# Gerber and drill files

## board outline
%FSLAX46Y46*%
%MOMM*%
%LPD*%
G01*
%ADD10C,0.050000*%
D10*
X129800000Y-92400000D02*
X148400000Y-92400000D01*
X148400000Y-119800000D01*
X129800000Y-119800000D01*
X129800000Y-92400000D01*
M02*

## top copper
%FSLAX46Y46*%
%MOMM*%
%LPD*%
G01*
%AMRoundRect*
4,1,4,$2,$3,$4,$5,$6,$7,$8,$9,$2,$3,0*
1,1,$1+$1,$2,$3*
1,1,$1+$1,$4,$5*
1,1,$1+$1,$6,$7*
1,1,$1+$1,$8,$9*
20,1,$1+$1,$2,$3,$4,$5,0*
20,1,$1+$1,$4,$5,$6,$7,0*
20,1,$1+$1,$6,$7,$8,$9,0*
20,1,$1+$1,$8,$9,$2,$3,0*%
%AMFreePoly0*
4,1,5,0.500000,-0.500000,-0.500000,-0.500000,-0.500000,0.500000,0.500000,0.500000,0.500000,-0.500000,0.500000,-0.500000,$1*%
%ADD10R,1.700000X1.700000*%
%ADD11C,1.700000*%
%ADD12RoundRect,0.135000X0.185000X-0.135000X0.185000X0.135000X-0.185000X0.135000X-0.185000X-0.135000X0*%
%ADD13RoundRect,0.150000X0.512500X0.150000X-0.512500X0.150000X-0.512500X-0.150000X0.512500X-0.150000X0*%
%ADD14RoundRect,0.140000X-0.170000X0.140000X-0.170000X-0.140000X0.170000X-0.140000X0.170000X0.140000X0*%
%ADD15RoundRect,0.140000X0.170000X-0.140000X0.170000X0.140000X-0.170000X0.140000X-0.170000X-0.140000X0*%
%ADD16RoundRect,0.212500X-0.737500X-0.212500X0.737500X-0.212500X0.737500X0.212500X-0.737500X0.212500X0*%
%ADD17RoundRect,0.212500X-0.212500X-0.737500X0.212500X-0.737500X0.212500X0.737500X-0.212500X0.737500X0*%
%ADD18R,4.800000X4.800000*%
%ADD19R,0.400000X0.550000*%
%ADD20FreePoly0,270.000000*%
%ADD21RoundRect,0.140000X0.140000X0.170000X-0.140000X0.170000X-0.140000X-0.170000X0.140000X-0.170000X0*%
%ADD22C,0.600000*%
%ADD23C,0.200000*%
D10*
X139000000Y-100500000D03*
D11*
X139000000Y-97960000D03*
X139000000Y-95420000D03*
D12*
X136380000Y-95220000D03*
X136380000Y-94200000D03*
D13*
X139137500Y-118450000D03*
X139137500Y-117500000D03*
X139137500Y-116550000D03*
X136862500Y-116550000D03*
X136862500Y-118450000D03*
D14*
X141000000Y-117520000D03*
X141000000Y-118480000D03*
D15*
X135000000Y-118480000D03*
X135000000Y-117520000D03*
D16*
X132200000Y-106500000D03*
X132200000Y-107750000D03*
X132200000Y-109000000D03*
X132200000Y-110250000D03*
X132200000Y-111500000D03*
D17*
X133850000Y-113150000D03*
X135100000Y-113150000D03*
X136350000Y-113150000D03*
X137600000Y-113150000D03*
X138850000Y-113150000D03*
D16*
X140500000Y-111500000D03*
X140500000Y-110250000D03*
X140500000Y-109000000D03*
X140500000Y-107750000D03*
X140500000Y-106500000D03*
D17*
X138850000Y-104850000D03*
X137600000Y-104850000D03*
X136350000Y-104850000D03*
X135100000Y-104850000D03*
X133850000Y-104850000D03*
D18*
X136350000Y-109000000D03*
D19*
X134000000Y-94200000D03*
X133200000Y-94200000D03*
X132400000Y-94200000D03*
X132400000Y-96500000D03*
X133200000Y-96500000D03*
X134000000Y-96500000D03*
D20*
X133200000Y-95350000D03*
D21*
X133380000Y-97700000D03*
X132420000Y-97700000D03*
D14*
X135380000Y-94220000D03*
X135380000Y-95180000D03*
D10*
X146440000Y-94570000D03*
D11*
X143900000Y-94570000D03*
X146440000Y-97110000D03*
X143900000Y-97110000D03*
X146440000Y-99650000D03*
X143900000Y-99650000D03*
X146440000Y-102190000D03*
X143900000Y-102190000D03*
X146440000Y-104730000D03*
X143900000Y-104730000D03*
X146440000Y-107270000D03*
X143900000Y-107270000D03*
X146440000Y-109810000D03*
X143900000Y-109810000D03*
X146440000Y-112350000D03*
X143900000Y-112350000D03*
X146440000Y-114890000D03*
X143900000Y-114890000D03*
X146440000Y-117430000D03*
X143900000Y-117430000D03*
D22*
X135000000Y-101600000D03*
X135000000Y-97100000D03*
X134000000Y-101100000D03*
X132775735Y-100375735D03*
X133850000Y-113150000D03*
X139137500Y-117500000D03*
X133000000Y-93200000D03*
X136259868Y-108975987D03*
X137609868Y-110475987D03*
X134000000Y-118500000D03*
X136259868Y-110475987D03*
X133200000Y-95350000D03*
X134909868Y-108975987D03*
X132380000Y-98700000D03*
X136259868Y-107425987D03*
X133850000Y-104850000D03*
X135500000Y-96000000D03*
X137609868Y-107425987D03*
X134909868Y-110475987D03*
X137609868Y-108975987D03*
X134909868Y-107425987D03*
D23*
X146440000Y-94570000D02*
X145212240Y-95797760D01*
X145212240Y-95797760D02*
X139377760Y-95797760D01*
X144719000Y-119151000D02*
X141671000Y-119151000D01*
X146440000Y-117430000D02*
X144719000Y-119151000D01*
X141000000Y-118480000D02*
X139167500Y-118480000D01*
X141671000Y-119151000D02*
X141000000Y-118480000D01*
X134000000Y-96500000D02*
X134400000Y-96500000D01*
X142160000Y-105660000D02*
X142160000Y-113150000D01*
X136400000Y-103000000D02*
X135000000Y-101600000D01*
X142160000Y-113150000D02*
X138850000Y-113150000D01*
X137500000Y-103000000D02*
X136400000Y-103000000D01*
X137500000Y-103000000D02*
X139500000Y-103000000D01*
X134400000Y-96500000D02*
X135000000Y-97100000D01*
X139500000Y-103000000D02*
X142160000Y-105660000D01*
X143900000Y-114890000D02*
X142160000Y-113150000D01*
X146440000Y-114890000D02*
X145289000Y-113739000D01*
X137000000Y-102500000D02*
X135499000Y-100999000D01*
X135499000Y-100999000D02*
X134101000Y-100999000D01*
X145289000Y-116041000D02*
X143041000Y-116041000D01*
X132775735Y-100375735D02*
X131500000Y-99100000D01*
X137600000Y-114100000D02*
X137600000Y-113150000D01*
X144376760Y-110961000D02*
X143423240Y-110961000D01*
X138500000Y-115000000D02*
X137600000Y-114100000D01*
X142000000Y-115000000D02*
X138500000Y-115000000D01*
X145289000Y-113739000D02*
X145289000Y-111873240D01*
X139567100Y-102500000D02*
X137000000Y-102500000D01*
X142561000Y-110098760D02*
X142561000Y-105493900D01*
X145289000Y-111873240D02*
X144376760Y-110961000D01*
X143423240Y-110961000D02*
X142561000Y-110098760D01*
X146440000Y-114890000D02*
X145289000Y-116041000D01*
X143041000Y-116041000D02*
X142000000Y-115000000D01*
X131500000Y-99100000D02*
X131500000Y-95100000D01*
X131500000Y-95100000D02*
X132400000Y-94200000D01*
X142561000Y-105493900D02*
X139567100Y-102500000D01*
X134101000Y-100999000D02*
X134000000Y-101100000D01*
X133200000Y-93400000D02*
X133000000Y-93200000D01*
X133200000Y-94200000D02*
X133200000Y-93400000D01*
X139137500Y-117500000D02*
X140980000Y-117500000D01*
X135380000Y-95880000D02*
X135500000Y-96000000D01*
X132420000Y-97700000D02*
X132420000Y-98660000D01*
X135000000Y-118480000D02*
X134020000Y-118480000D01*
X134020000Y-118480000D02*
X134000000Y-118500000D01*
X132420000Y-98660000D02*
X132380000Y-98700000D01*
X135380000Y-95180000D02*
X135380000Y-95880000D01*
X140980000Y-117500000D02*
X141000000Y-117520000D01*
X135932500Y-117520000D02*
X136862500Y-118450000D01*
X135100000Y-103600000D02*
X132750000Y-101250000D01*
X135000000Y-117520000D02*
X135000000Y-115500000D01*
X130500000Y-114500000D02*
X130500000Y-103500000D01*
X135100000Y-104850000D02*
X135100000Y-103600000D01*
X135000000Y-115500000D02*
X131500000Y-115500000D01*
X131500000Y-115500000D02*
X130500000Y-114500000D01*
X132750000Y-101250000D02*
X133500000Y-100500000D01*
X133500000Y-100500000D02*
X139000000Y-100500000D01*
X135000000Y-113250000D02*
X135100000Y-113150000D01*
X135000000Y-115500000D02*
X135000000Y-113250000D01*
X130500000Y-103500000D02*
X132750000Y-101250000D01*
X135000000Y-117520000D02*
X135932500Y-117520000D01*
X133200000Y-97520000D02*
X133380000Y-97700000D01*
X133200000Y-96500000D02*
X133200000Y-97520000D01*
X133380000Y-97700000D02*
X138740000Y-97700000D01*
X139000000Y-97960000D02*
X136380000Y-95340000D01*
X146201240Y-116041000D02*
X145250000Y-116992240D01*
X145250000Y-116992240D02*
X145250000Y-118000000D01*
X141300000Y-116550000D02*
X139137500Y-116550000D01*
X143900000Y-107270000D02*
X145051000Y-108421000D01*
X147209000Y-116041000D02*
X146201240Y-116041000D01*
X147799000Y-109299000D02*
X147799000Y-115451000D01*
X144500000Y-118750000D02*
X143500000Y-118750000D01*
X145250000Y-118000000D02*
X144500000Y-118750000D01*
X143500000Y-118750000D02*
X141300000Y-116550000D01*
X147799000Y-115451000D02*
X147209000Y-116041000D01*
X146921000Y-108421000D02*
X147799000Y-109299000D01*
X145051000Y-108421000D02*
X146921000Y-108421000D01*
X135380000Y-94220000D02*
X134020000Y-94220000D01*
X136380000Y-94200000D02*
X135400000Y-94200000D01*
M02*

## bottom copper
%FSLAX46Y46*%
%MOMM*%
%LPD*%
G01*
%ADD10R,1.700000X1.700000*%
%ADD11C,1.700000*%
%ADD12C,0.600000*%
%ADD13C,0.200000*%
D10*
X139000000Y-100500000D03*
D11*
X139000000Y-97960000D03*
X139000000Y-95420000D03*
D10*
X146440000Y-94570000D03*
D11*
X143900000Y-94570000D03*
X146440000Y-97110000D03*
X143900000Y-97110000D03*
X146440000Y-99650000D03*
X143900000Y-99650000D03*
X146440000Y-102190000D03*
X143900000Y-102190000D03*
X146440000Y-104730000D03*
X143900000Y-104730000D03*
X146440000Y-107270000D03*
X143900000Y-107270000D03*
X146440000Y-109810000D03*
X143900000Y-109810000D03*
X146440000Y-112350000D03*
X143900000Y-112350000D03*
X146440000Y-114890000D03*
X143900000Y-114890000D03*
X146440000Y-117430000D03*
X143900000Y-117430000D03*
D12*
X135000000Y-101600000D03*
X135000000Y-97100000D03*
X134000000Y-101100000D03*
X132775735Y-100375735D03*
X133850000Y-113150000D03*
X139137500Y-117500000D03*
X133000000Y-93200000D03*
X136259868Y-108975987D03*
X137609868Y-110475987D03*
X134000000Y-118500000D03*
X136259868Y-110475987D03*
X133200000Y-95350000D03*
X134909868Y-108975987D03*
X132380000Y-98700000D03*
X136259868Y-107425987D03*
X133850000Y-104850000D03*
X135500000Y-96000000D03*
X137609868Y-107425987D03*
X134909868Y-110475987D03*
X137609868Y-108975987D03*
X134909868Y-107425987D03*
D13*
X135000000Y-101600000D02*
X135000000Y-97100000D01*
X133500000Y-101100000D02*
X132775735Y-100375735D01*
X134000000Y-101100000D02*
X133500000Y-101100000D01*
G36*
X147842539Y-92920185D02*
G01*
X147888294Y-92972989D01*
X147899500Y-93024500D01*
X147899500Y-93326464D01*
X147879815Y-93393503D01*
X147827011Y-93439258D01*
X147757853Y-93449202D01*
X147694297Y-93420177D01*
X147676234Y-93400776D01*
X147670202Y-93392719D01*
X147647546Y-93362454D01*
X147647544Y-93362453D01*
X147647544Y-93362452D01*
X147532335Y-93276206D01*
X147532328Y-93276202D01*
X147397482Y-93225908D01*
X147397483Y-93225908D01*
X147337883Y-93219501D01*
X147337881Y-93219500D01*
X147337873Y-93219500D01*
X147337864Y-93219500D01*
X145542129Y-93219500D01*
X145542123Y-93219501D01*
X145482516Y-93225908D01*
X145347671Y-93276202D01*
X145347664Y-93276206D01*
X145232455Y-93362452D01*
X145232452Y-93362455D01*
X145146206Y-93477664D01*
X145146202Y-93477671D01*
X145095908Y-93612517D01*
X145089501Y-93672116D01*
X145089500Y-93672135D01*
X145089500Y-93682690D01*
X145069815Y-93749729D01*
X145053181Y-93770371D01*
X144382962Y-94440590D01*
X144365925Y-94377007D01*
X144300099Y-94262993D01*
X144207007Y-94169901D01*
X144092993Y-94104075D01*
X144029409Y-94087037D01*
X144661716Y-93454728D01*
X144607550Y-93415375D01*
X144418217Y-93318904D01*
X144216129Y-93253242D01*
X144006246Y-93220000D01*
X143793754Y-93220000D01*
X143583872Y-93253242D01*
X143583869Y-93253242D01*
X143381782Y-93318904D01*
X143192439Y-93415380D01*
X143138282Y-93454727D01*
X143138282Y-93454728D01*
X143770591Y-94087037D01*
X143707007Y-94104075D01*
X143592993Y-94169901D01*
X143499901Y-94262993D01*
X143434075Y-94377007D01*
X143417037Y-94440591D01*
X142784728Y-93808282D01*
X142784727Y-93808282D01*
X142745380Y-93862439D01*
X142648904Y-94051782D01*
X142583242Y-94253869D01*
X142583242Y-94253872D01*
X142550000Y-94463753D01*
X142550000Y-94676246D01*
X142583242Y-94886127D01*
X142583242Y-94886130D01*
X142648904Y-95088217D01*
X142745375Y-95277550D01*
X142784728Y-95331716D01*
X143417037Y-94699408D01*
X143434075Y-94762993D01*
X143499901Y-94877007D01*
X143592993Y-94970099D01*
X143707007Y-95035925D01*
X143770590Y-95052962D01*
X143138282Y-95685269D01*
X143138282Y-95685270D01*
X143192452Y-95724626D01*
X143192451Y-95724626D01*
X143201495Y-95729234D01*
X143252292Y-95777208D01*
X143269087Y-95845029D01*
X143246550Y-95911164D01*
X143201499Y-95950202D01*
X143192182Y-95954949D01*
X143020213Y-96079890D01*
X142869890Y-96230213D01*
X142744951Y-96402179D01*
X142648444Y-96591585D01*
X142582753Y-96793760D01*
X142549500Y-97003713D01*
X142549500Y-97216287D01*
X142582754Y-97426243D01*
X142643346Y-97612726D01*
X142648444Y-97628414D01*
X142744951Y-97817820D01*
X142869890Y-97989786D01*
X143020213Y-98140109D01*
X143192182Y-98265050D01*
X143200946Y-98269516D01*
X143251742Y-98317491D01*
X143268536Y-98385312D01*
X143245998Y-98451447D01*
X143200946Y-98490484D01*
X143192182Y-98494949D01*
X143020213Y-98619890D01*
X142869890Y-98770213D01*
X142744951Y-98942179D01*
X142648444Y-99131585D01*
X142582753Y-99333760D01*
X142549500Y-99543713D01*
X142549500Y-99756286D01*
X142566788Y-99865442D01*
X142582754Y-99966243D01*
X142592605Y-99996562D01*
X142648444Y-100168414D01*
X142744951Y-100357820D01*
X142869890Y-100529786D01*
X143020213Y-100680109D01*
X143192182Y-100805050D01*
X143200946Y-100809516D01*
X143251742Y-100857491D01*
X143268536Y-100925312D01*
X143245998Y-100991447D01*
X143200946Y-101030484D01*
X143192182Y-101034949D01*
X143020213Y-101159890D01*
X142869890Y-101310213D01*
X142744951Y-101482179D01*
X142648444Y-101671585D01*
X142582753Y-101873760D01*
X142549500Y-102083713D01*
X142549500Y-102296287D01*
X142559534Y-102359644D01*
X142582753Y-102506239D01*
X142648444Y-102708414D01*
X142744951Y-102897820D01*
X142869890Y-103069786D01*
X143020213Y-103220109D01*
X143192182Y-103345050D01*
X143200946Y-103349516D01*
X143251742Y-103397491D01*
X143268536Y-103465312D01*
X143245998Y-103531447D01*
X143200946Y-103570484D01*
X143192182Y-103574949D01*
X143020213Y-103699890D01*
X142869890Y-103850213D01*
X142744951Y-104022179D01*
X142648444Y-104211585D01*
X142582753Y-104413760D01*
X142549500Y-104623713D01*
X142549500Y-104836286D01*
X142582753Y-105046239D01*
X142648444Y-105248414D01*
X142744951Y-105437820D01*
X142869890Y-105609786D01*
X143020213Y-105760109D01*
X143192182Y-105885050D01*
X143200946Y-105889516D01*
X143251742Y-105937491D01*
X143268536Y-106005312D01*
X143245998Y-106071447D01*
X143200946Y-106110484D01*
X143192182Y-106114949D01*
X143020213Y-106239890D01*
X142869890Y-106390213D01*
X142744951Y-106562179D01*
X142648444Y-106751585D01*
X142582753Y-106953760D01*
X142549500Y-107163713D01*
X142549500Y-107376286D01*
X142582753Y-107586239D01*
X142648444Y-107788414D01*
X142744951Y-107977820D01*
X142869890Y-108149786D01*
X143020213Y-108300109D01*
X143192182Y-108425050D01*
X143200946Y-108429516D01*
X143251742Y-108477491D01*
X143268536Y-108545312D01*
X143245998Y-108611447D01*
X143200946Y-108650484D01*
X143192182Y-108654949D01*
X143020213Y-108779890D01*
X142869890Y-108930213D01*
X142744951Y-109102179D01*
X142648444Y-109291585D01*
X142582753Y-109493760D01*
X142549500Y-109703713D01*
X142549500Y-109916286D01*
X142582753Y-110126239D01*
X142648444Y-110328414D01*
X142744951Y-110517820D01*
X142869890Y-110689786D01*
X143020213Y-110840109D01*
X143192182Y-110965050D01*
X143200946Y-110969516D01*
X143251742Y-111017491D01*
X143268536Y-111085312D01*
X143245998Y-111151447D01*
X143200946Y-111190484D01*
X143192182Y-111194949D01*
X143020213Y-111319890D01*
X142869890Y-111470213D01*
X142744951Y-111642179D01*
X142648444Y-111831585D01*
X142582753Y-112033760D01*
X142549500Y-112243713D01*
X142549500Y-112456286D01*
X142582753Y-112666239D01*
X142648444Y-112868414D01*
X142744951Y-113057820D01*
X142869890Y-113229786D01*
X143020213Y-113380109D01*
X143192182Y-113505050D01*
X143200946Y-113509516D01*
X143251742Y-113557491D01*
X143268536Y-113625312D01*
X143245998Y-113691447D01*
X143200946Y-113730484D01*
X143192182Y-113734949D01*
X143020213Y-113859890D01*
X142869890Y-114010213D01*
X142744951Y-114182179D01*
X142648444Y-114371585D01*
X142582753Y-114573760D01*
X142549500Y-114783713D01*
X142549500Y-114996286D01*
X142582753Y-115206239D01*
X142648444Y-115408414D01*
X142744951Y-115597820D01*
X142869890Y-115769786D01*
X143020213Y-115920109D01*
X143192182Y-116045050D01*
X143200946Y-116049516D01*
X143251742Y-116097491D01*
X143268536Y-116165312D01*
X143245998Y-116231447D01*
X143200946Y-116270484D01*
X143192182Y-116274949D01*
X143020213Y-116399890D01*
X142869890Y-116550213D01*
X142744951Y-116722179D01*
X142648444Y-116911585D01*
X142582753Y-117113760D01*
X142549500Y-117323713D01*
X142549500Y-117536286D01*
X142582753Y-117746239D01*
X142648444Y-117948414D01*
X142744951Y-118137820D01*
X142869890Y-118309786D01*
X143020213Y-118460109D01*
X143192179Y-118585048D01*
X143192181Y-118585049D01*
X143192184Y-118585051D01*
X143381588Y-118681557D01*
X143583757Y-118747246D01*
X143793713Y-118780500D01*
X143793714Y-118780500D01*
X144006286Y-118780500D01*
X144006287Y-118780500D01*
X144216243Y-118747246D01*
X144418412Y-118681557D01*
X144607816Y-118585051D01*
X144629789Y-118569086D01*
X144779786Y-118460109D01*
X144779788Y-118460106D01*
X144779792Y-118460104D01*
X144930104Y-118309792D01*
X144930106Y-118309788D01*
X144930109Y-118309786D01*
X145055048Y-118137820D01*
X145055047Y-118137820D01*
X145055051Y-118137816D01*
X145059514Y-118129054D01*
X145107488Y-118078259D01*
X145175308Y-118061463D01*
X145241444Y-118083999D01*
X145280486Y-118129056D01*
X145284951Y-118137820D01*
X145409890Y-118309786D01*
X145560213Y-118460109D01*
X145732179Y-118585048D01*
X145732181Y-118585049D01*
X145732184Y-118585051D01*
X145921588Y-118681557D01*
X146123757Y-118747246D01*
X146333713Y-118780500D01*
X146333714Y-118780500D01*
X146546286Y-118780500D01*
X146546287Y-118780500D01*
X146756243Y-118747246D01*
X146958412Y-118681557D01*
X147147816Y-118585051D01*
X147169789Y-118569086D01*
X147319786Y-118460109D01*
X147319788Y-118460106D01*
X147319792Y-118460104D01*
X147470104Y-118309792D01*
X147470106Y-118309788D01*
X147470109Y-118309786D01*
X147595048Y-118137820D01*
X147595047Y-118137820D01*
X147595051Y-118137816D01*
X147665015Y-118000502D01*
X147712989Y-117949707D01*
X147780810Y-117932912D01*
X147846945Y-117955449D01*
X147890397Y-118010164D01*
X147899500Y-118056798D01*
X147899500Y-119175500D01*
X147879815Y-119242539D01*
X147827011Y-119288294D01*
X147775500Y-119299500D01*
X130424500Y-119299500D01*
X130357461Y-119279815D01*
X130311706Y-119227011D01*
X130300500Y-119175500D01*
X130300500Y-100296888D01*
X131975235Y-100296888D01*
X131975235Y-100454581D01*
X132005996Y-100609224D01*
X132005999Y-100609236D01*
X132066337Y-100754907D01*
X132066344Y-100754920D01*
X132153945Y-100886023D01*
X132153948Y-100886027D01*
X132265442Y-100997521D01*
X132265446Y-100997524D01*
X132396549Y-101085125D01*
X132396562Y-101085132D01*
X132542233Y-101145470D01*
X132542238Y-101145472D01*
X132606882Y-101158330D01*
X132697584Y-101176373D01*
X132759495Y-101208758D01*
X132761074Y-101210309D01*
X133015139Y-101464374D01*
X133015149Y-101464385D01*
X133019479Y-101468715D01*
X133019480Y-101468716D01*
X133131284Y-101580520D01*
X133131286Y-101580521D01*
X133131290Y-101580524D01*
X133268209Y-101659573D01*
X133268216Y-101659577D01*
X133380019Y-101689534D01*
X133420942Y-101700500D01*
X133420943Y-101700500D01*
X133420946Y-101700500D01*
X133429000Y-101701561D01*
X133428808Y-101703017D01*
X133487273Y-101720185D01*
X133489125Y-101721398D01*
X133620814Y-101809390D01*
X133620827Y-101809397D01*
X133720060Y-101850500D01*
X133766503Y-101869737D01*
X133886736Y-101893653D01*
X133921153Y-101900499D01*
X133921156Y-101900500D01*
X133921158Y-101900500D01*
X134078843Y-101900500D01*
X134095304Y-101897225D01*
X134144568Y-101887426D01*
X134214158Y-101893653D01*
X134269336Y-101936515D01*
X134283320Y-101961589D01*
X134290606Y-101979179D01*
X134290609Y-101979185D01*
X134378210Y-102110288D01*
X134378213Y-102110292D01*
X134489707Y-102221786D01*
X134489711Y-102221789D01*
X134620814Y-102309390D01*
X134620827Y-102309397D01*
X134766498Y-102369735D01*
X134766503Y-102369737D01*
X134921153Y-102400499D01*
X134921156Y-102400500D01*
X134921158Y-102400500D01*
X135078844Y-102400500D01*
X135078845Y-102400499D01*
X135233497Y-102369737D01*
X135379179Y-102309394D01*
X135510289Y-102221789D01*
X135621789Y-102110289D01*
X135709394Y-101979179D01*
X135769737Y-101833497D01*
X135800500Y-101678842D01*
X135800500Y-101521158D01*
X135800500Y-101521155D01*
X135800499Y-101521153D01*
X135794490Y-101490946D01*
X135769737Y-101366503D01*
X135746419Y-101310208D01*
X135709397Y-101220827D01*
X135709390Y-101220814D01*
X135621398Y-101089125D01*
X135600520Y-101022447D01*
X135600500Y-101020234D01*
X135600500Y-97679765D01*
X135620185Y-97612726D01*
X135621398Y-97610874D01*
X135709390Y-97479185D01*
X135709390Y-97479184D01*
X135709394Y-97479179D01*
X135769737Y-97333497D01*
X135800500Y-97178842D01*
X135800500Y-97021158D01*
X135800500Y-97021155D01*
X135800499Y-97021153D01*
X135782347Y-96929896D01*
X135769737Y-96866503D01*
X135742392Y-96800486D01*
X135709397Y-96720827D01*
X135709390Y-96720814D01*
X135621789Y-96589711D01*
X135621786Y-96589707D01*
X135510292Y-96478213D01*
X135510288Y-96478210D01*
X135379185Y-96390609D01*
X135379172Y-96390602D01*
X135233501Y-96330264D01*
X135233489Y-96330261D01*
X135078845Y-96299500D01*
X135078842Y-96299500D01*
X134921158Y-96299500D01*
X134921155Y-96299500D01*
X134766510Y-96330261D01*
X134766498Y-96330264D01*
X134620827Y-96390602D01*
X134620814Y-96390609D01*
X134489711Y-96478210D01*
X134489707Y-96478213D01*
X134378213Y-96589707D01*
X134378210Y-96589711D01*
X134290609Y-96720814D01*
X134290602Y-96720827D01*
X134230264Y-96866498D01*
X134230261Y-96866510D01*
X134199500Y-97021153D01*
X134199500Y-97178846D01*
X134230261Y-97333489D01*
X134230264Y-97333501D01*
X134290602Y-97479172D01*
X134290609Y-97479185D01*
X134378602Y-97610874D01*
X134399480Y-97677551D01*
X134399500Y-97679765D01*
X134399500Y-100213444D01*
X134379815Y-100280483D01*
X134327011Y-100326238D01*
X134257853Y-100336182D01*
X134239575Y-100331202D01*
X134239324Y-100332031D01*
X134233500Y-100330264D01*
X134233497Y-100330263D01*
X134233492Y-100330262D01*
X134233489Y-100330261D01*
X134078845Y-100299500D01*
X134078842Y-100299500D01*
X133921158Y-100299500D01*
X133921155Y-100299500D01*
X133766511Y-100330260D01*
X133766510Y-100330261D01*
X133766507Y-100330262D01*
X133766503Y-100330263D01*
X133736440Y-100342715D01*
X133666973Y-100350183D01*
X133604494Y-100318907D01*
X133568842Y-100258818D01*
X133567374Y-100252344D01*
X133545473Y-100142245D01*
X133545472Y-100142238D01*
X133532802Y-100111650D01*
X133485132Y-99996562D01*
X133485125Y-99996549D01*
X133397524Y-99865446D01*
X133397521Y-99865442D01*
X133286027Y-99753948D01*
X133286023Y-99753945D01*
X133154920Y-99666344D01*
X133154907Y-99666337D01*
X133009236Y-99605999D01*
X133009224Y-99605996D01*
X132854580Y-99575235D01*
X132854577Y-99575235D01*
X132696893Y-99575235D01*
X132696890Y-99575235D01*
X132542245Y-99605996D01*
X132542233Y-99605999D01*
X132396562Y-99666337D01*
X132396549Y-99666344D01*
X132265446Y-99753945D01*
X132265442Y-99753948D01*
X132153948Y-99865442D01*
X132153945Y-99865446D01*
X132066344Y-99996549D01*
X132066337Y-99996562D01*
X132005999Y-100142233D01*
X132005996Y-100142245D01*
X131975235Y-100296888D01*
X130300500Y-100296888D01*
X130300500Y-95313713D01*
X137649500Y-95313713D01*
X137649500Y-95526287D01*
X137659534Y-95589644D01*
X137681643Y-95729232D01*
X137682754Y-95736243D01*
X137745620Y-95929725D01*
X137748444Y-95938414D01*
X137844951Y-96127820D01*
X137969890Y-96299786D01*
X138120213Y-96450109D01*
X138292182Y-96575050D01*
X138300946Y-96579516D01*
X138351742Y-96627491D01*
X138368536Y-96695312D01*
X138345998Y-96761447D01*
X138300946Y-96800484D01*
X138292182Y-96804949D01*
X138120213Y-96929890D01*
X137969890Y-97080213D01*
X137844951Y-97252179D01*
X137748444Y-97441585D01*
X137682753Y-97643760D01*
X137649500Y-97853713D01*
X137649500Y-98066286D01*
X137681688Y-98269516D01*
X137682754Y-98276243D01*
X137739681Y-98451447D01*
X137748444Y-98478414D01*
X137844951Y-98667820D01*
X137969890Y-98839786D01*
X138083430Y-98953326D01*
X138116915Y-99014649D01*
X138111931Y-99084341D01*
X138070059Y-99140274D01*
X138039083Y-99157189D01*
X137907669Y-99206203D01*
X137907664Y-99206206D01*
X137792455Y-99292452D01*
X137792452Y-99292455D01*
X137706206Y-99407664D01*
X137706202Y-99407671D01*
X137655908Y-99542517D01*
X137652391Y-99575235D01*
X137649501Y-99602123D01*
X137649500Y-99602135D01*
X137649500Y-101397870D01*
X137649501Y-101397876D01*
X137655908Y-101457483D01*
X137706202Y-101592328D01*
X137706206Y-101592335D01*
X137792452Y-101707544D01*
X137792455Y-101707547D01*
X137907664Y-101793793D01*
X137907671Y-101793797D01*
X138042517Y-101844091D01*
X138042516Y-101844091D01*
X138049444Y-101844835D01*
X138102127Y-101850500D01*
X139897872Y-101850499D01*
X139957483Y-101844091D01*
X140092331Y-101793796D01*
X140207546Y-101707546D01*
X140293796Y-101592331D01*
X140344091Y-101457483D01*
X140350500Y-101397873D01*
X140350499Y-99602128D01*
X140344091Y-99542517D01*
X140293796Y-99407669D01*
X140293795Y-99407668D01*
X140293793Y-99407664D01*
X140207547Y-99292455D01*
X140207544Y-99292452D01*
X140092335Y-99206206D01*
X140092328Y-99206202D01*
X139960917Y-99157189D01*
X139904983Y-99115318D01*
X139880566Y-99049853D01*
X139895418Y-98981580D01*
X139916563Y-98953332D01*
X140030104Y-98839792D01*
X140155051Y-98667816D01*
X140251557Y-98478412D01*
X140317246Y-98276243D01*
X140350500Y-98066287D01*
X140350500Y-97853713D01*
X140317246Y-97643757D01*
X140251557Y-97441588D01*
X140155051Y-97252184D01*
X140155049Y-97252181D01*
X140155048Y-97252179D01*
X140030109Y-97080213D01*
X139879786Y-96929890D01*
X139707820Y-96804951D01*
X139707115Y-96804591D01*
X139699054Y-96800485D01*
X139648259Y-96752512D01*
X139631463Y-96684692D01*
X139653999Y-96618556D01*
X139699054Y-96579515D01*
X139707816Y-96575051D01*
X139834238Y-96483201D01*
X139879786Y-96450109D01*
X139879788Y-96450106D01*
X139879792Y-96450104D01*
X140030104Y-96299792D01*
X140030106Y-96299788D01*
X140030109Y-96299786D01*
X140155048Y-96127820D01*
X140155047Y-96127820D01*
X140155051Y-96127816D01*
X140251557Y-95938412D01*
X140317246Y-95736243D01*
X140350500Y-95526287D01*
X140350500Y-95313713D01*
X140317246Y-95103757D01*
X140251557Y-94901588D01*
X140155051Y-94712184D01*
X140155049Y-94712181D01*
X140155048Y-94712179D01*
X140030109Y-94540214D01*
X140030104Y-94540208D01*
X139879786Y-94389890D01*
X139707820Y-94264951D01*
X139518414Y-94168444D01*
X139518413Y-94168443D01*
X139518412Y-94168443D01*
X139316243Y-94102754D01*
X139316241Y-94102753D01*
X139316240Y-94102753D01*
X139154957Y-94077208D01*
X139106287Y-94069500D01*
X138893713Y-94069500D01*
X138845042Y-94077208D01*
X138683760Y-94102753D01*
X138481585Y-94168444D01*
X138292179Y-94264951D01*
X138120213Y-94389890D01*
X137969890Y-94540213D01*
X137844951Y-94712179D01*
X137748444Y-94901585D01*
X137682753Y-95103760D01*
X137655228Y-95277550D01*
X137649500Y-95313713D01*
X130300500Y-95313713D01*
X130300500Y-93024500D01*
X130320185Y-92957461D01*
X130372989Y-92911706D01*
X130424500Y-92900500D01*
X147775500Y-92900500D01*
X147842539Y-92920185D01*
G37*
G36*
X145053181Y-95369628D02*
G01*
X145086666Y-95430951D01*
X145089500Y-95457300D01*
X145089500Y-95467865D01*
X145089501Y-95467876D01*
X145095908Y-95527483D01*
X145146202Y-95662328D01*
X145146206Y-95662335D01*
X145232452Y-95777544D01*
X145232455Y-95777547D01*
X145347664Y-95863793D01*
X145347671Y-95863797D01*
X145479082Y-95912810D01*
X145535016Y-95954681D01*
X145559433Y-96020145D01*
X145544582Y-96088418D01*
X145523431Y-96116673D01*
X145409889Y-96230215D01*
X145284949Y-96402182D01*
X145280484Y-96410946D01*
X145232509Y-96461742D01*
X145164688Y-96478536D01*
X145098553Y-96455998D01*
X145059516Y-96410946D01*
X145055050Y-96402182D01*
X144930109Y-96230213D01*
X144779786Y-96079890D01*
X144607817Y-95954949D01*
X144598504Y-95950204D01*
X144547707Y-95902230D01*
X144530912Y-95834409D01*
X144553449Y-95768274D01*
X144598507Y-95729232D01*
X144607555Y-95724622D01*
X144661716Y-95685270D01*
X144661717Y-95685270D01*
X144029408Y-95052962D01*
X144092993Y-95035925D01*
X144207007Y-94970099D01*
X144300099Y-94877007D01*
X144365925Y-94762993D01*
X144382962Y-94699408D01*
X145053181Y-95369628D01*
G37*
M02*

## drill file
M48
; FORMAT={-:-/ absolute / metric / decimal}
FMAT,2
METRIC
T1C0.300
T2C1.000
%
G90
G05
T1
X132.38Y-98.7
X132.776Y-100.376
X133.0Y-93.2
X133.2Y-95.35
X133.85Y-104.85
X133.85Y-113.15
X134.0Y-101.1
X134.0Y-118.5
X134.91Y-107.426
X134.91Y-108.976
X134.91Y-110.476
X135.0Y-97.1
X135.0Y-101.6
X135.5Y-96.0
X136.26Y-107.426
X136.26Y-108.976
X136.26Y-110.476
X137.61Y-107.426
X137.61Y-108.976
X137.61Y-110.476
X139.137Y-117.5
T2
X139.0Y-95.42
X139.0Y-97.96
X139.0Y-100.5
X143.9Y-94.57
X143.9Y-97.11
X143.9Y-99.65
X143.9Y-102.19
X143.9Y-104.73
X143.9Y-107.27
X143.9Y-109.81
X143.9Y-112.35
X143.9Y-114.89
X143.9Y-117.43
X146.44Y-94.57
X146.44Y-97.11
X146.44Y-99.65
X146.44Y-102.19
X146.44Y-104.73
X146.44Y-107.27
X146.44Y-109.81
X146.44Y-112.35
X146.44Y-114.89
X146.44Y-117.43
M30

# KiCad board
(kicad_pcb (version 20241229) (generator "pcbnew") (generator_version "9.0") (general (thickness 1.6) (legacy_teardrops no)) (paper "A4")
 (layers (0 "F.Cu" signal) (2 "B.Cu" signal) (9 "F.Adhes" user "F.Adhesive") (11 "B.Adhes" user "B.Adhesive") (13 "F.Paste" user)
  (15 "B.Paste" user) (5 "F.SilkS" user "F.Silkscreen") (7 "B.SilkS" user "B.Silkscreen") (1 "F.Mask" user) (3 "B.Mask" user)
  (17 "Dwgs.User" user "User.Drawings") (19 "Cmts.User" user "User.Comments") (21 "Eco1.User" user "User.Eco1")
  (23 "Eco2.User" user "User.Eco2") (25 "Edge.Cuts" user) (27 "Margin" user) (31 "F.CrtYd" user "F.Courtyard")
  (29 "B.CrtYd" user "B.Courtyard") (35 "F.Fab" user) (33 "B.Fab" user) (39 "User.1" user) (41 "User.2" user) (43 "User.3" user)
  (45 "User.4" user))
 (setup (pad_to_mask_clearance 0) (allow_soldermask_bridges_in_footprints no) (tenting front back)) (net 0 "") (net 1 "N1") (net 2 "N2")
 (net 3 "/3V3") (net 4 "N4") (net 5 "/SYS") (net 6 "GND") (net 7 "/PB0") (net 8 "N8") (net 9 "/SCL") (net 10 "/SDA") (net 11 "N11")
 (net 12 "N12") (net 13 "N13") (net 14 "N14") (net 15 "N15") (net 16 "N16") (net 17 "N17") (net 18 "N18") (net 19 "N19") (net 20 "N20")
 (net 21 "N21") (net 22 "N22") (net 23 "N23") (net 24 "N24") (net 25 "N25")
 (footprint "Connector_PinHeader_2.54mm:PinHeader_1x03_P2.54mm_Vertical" (layer "F.Cu") (at 139 100.5 180)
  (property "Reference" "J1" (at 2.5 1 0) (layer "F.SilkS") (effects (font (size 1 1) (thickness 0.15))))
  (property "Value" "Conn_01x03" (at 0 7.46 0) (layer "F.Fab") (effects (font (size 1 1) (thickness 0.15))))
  (pad "1" thru_hole rect (at 0 0 180) (size 1.7 1.7) (drill 1) (layers "*.Cu" "*.Mask") (remove_unused_layers no) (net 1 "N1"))
  (pad "2" thru_hole circle (at 0 2.54 180) (size 1.7 1.7) (drill 1) (layers "*.Cu" "*.Mask") (remove_unused_layers no) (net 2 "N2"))
  (pad "3" thru_hole circle (at 0 5.08 180) (size 1.7 1.7) (drill 1) (layers "*.Cu" "*.Mask") (remove_unused_layers no) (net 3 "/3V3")))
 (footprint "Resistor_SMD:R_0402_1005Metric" (layer "F.Cu") (at 136.38 94.71 90)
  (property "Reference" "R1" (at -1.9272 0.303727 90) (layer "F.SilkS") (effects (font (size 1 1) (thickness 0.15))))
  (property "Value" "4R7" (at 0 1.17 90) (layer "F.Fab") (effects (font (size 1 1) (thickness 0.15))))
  (pad "1" smd roundrect (at -0.51 0 90) (size 0.54 0.64) (layers "F.Cu" "F.Mask" "F.Paste") (roundrect_rratio 0.25) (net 2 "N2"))
  (pad "2" smd roundrect (at 0.51 0 90) (size 0.54 0.64) (layers "F.Cu" "F.Mask" "F.Paste") (roundrect_rratio 0.25) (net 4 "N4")))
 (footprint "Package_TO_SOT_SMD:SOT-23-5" (layer "F.Cu") (at 138 117.5 180)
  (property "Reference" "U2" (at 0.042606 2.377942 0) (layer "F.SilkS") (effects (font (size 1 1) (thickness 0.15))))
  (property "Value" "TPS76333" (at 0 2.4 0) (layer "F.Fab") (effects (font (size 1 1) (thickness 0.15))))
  (pad "1" smd roundrect (at -1.1375 -0.95 180) (size 1.325 0.6) (layers "F.Cu" "F.Mask" "F.Paste") (roundrect_rratio 0.25) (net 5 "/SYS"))
  (pad "2" smd roundrect (at -1.1375 0 180) (size 1.325 0.6) (layers "F.Cu" "F.Mask" "F.Paste") (roundrect_rratio 0.25) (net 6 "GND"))
  (pad "3" smd roundrect (at -1.1375 0.95 180) (size 1.325 0.6) (layers "F.Cu" "F.Mask" "F.Paste") (roundrect_rratio 0.25) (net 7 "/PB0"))
  (pad "4" smd roundrect (at 1.1375 0.95 180) (size 1.325 0.6) (layers "F.Cu" "F.Mask" "F.Paste") (roundrect_rratio 0.25) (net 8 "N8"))
  (pad "5" smd roundrect (at 1.1375 -0.95 180) (size 1.325 0.6) (layers "F.Cu" "F.Mask" "F.Paste") (roundrect_rratio 0.25) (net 1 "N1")))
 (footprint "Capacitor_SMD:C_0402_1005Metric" (layer "F.Cu") (at 141 118 -90)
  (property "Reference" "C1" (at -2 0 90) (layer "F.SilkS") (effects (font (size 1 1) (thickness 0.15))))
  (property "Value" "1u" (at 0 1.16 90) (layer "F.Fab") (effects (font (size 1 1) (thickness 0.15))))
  (pad "1" smd roundrect (at -0.48 0 270) (size 0.56 0.62) (layers "F.Cu" "F.Mask" "F.Paste") (roundrect_rratio 0.25) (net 6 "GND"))
  (pad "2" smd roundrect (at 0.48 0 270) (size 0.56 0.62) (layers "F.Cu" "F.Mask" "F.Paste") (roundrect_rratio 0.25) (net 5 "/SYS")))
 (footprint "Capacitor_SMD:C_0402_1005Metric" (layer "F.Cu") (at 135 118 90)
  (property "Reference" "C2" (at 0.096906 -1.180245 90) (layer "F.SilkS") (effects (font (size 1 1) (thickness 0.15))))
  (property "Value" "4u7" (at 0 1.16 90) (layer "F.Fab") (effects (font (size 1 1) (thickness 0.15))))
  (pad "1" smd roundrect (at -0.48 0 90) (size 0.56 0.62) (layers "F.Cu" "F.Mask" "F.Paste") (roundrect_rratio 0.25) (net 6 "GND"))
  (pad "2" smd roundrect (at 0.48 0 90) (size 0.56 0.62) (layers "F.Cu" "F.Mask" "F.Paste") (roundrect_rratio 0.25) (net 1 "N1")))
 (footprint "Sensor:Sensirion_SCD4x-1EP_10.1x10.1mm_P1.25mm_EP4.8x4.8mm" (layer "F.Cu") (at 136.35 109)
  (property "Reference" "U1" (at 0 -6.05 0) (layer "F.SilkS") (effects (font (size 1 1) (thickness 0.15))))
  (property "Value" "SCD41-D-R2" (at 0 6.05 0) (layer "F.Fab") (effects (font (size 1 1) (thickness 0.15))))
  (pad "" smd roundrect (at -1.2 -1.2) (size 1.93 1.93) (layers "F.Paste") (roundrect_rratio 0.129534))
  (pad "" smd roundrect (at -1.2 1.2) (size 1.93 1.93) (layers "F.Paste") (roundrect_rratio 0.129534))
  (pad "" smd roundrect (at 1.2 -1.2) (size 1.93 1.93) (layers "F.Paste") (roundrect_rratio 0.129534))
  (pad "" smd roundrect (at 1.2 1.2) (size 1.93 1.93) (layers "F.Paste") (roundrect_rratio 0.129534))
  (pad "1" smd roundrect (at -4.15 -2.5) (size 1.9 0.85) (layers "F.Cu" "F.Mask" "F.Paste") (roundrect_rratio 0.25))
  (pad "2" smd roundrect (at -4.15 -1.25) (size 1.9 0.85) (layers "F.Cu" "F.Mask" "F.Paste") (roundrect_rratio 0.25))
  (pad "3" smd roundrect (at -4.15 0) (size 1.9 0.85) (layers "F.Cu" "F.Mask" "F.Paste") (roundrect_rratio 0.25))
  (pad "4" smd roundrect (at -4.15 1.25) (size 1.9 0.85) (layers "F.Cu" "F.Mask" "F.Paste") (roundrect_rratio 0.25))
  (pad "5" smd roundrect (at -4.15 2.5) (size 1.9 0.85) (layers "F.Cu" "F.Mask" "F.Paste") (roundrect_rratio 0.25))
  (pad "6" smd roundrect (at -2.5 4.15) (size 0.85 1.9) (layers "F.Cu" "F.Mask" "F.Paste") (roundrect_rratio 0.25) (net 6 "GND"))
  (pad "7" smd roundrect (at -1.25 4.15) (size 0.85 1.9) (layers "F.Cu" "F.Mask" "F.Paste") (roundrect_rratio 0.25) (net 1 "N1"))
  (pad "8" smd roundrect (at 0 4.15) (size 0.85 1.9) (layers "F.Cu" "F.Mask" "F.Paste") (roundrect_rratio 0.25))
  (pad "9" smd roundrect (at 1.25 4.15) (size 0.85 1.9) (layers "F.Cu" "F.Mask" "F.Paste") (roundrect_rratio 0.25) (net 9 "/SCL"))
  (pad "10" smd roundrect (at 2.5 4.15) (size 0.85 1.9) (layers "F.Cu" "F.Mask" "F.Paste") (roundrect_rratio 0.25) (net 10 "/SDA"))
  (pad "11" smd roundrect (at 4.15 2.5) (size 1.9 0.85) (layers "F.Cu" "F.Mask" "F.Paste") (roundrect_rratio 0.25))
  (pad "12" smd roundrect (at 4.15 1.25) (size 1.9 0.85) (layers "F.Cu" "F.Mask" "F.Paste") (roundrect_rratio 0.25))
  (pad "13" smd roundrect (at 4.15 0) (size 1.9 0.85) (layers "F.Cu" "F.Mask" "F.Paste") (roundrect_rratio 0.25))
  (pad "14" smd roundrect (at 4.15 -1.25) (size 1.9 0.85) (layers "F.Cu" "F.Mask" "F.Paste") (roundrect_rratio 0.25))
  (pad "15" smd roundrect (at 4.15 -2.5) (size 1.9 0.85) (layers "F.Cu" "F.Mask" "F.Paste") (roundrect_rratio 0.25))
  (pad "16" smd roundrect (at 2.5 -4.15) (size 0.85 1.9) (layers "F.Cu" "F.Mask" "F.Paste") (roundrect_rratio 0.25))
  (pad "17" smd roundrect (at 1.25 -4.15) (size 0.85 1.9) (layers "F.Cu" "F.Mask" "F.Paste") (roundrect_rratio 0.25))
  (pad "18" smd roundrect (at 0 -4.15) (size 0.85 1.9) (layers "F.Cu" "F.Mask" "F.Paste") (roundrect_rratio 0.25))
  (pad "19" smd roundrect (at -1.25 -4.15) (size 0.85 1.9) (layers "F.Cu" "F.Mask" "F.Paste") (roundrect_rratio 0.25) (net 1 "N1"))
  (pad "20" smd roundrect (at -2.5 -4.15) (size 0.85 1.9) (layers "F.Cu" "F.Mask" "F.Paste") (roundrect_rratio 0.25) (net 6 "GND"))
  (pad "21" smd rect (at 0 0) (size 4.8 4.8) (layers "F.Cu" "F.Mask") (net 6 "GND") (zone_connect 2)))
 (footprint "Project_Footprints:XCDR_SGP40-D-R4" (layer "F.Cu") (at 133.2 95.35 -90)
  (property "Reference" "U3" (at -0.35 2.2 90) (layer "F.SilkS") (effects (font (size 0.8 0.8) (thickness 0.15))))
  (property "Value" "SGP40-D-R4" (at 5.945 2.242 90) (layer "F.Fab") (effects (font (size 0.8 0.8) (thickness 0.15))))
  (pad "1" smd rect (at -1.15 -0.8 270) (size 0.55 0.4) (layers "F.Cu" "F.Mask" "F.Paste") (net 4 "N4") (solder_mask_margin 0.102))
  (pad "2" smd rect (at -1.15 0 270) (size 0.55 0.4) (layers "F.Cu" "F.Mask" "F.Paste") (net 6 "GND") (solder_mask_margin 0.102))
  (pad "3" smd rect (at -1.15 0.8 270) (size 0.55 0.4) (layers "F.Cu" "F.Mask" "F.Paste") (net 9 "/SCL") (solder_mask_margin 0.102))
  (pad "4" smd rect (at 1.15 0.8 270) (size 0.55 0.4) (layers "F.Cu" "F.Mask" "F.Paste") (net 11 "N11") (solder_mask_margin 0.102))
  (pad "5" smd rect (at 1.15 0 270) (size 0.55 0.4) (layers "F.Cu" "F.Mask" "F.Paste") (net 2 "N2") (solder_mask_margin 0.102))
  (pad "6" smd rect (at 1.15 -0.8 270) (size 0.55 0.4) (layers "F.Cu" "F.Mask" "F.Paste") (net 10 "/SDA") (solder_mask_margin 0.102))
  (pad "7" smd custom (at 0 0 270) (size 1 1) (layers "F.Cu") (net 6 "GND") (options (clearance outline) (anchor rect)) (primitives)))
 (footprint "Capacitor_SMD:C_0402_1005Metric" (layer "F.Cu") (at 132.9 97.7 180)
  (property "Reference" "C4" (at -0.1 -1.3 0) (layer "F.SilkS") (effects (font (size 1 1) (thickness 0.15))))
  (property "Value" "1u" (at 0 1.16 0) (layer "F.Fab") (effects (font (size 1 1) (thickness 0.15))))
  (pad "1" smd roundrect (at -0.48 0 180) (size 0.56 0.62) (layers "F.Cu" "F.Mask" "F.Paste") (roundrect_rratio 0.25) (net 2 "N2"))
  (pad "2" smd roundrect (at 0.48 0 180) (size 0.56 0.62) (layers "F.Cu" "F.Mask" "F.Paste") (roundrect_rratio 0.25) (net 6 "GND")))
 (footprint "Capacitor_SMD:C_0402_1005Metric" (layer "F.Cu") (at 135.38 94.7 -90)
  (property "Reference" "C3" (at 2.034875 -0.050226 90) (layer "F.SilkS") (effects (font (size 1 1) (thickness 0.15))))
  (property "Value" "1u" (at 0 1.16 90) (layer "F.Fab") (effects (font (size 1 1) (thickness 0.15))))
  (pad "1" smd roundrect (at -0.48 0 270) (size 0.56 0.62) (layers "F.Cu" "F.Mask" "F.Paste") (roundrect_rratio 0.25) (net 4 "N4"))
  (pad "2" smd roundrect (at 0.48 0 270) (size 0.56 0.62) (layers "F.Cu" "F.Mask" "F.Paste") (roundrect_rratio 0.25) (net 6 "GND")))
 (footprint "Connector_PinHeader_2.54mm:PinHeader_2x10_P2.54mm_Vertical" (layer "B.Cu") (at 146.44 94.57 180)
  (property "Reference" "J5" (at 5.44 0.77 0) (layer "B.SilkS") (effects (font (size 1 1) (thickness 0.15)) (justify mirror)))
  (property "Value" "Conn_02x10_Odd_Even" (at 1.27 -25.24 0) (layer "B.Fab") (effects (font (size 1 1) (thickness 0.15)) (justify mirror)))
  (pad "1" thru_hole rect (at 0 0 180) (size 1.7 1.7) (drill 1) (layers "*.Cu" "*.Mask") (remove_unused_layers no) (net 3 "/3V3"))
  (pad "2" thru_hole circle (at 2.54 0 180) (size 1.7 1.7) (drill 1) (layers "*.Cu" "*.Mask") (remove_unused_layers no) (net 6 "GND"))
  (pad "3" thru_hole circle (at 0 -2.54 180) (size 1.7 1.7) (drill 1) (layers "*.Cu" "*.Mask") (remove_unused_layers no) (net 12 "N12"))
  (pad "4" thru_hole circle (at 2.54 -2.54 180) (size 1.7 1.7) (drill 1) (layers "*.Cu" "*.Mask") (remove_unused_layers no) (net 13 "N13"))
  (pad "5" thru_hole circle (at 0 -5.08 180) (size 1.7 1.7) (drill 1) (layers "*.Cu" "*.Mask") (remove_unused_layers no) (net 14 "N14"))
  (pad "6" thru_hole circle (at 2.54 -5.08 180) (size 1.7 1.7) (drill 1) (layers "*.Cu" "*.Mask") (remove_unused_layers no) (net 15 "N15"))
  (pad "7" thru_hole circle (at 0 -7.62 180) (size 1.7 1.7) (drill 1) (layers "*.Cu" "*.Mask") (remove_unused_layers no) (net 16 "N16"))
  (pad "8" thru_hole circle (at 2.54 -7.62 180) (size 1.7 1.7) (drill 1) (layers "*.Cu" "*.Mask") (remove_unused_layers no) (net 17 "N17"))
  (pad "9" thru_hole circle (at 0 -10.16 180) (size 1.7 1.7) (drill 1) (layers "*.Cu" "*.Mask") (remove_unused_layers no) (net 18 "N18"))
  (pad "10" thru_hole circle (at 2.54 -10.16 180) (size 1.7 1.7) (drill 1) (layers "*.Cu" "*.Mask") (remove_unused_layers no) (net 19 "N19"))
  (pad "11" thru_hole circle (at 0 -12.7 180) (size 1.7 1.7) (drill 1) (layers "*.Cu" "*.Mask") (remove_unused_layers no) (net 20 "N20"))
  (pad "12" thru_hole circle (at 2.54 -12.7 180) (size 1.7 1.7) (drill 1) (layers "*.Cu" "*.Mask") (remove_unused_layers no) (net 7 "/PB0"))
  (pad "13" thru_hole circle (at 0 -15.24 180) (size 1.7 1.7) (drill 1) (layers "*.Cu" "*.Mask") (remove_unused_layers no) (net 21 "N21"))
  (pad "14" thru_hole circle (at 2.54 -15.24 180) (size 1.7 1.7) (drill 1) (layers "*.Cu" "*.Mask") (remove_unused_layers no) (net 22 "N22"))
  (pad "15" thru_hole circle (at 0 -17.78 180) (size 1.7 1.7) (drill 1) (layers "*.Cu" "*.Mask") (remove_unused_layers no) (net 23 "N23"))
  (pad "16" thru_hole circle (at 2.54 -17.78 180) (size 1.7 1.7) (drill 1) (layers "*.Cu" "*.Mask") (remove_unused_layers no) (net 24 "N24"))
  (pad "17" thru_hole circle (at 0 -20.32 180) (size 1.7 1.7) (drill 1) (layers "*.Cu" "*.Mask") (remove_unused_layers no) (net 9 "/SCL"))
  (pad "18" thru_hole circle (at 2.54 -20.32 180) (size 1.7 1.7) (drill 1) (layers "*.Cu" "*.Mask") (remove_unused_layers no)
   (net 10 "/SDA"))
  (pad "19" thru_hole circle (at 0 -22.86 180) (size 1.7 1.7) (drill 1) (layers "*.Cu" "*.Mask") (remove_unused_layers no) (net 5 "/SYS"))
  (pad "20" thru_hole circle (at 2.54 -22.86 180) (size 1.7 1.7) (drill 1) (layers "*.Cu" "*.Mask") (remove_unused_layers no) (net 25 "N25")))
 (gr_rect (start 129.8 92.4) (end 148.4 119.8) (stroke (width 0.05) (type default)) (fill no) (layer "Edge.Cuts"))
 (segment (start 146.44 94.57) (end 145.21224 95.79776) (width 0.2) (layer "F.Cu") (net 3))
 (segment (start 145.21224 95.79776) (end 139.37776 95.79776) (width 0.2) (layer "F.Cu") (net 3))
 (segment (start 144.719 119.151) (end 141.671 119.151) (width 0.2) (layer "F.Cu") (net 5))
 (segment (start 146.44 117.43) (end 144.719 119.151) (width 0.2) (layer "F.Cu") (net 5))
 (segment (start 141 118.48) (end 139.1675 118.48) (width 0.2) (layer "F.Cu") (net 5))
 (segment (start 141.671 119.151) (end 141 118.48) (width 0.2) (layer "F.Cu") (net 5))
 (segment (start 134 96.5) (end 134.4 96.5) (width 0.2) (layer "F.Cu") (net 10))
 (segment (start 142.16 105.66) (end 142.16 113.15) (width 0.2) (layer "F.Cu") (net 10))
 (segment (start 136.4 103) (end 135 101.6) (width 0.2) (layer "F.Cu") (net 10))
 (segment (start 142.16 113.15) (end 138.85 113.15) (width 0.2) (layer "F.Cu") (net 10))
 (segment (start 137.5 103) (end 136.4 103) (width 0.2) (layer "F.Cu") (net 10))
 (segment (start 137.5 103) (end 139.5 103) (width 0.2) (layer "F.Cu") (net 10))
 (segment (start 134.4 96.5) (end 135 97.1) (width 0.2) (layer "F.Cu") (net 10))
 (segment (start 139.5 103) (end 142.16 105.66) (width 0.2) (layer "F.Cu") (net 10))
 (segment (start 143.9 114.89) (end 142.16 113.15) (width 0.2) (layer "F.Cu") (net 10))
 (via (at 135 101.6) (size 0.6) (drill 0.3) (layers "F.Cu" "B.Cu") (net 10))
 (via (at 135 97.1) (size 0.6) (drill 0.3) (layers "F.Cu" "B.Cu") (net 10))
 (segment (start 135 101.6) (end 135 97.1) (width 0.2) (layer "B.Cu") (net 10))
 (segment (start 146.44 114.89) (end 145.289 113.739) (width 0.2) (layer "F.Cu") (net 9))
 (segment (start 137 102.5) (end 135.499 100.999) (width 0.2) (layer "F.Cu") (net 9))
 (segment (start 135.499 100.999) (end 134.101 100.999) (width 0.2) (layer "F.Cu") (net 9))
 (segment (start 145.289 116.041) (end 143.041 116.041) (width 0.2) (layer "F.Cu") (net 9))
 (segment (start 132.775735 100.375735) (end 131.5 99.1) (width 0.2) (layer "F.Cu") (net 9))
 (segment (start 137.6 114.1) (end 137.6 113.15) (width 0.2) (layer "F.Cu") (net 9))
 (segment (start 144.37676 110.961) (end 143.42324 110.961) (width 0.2) (layer "F.Cu") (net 9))
 (segment (start 138.5 115) (end 137.6 114.1) (width 0.2) (layer "F.Cu") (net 9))
 (segment (start 142 115) (end 138.5 115) (width 0.2) (layer "F.Cu") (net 9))
 (segment (start 145.289 113.739) (end 145.289 111.87324) (width 0.2) (layer "F.Cu") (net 9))
 (segment (start 139.5671 102.5) (end 137 102.5) (width 0.2) (layer "F.Cu") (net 9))
 (segment (start 142.561 110.09876) (end 142.561 105.4939) (width 0.2) (layer "F.Cu") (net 9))
 (segment (start 145.289 111.87324) (end 144.37676 110.961) (width 0.2) (layer "F.Cu") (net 9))
 (segment (start 143.42324 110.961) (end 142.561 110.09876) (width 0.2) (layer "F.Cu") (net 9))
 (segment (start 146.44 114.89) (end 145.289 116.041) (width 0.2) (layer "F.Cu") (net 9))
 (segment (start 143.041 116.041) (end 142 115) (width 0.2) (layer "F.Cu") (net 9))
 (segment (start 131.5 99.1) (end 131.5 95.1) (width 0.2) (layer "F.Cu") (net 9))
 (segment (start 131.5 95.1) (end 132.4 94.2) (width 0.2) (layer "F.Cu") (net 9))
 (segment (start 142.561 105.4939) (end 139.5671 102.5) (width 0.2) (layer "F.Cu") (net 9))
 (segment (start 134.101 100.999) (end 134 101.1) (width 0.2) (layer "F.Cu") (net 9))
 (via (at 134 101.1) (size 0.6) (drill 0.3) (layers "F.Cu" "B.Cu") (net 9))
 (via (at 132.775735 100.375735) (size 0.6) (drill 0.3) (layers "F.Cu" "B.Cu") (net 9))
 (segment (start 133.5 101.1) (end 132.775735 100.375735) (width 0.2) (layer "B.Cu") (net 9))
 (segment (start 134 101.1) (end 133.5 101.1) (width 0.2) (layer "B.Cu") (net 9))
 (segment (start 133.2 93.4) (end 133 93.2) (width 0.2) (layer "F.Cu") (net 6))
 (segment (start 133.2 94.2) (end 133.2 93.4) (width 0.2) (layer "F.Cu") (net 6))
 (segment (start 139.1375 117.5) (end 140.98 117.5) (width 0.2) (layer "F.Cu") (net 6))
 (segment (start 135.38 95.88) (end 135.5 96) (width 0.2) (layer "F.Cu") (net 6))
 (segment (start 132.42 97.7) (end 132.42 98.66) (width 0.2) (layer "F.Cu") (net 6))
 (segment (start 135 118.48) (end 134.02 118.48) (width 0.2) (layer "F.Cu") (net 6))
 (segment (start 134.02 118.48) (end 134 118.5) (width 0.2) (layer "F.Cu") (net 6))
 (segment (start 132.42 98.66) (end 132.38 98.7) (width 0.2) (layer "F.Cu") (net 6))
 (segment (start 135.38 95.18) (end 135.38 95.88) (width 0.2) (layer "F.Cu") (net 6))
 (segment (start 140.98 117.5) (end 141 117.52) (width 0.2) (layer "F.Cu") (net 6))
 (via (at 133.85 113.15) (size 0.6) (drill 0.3) (layers "F.Cu" "B.Cu") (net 6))
 (via (at 139.1375 117.5) (size 0.6) (drill 0.3) (layers "F.Cu" "B.Cu") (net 6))
 (via (at 133 93.2) (size 0.6) (drill 0.3) (layers "F.Cu" "B.Cu") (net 6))
 (via (at 136.259868 108.975987) (size 0.6) (drill 0.3) (layers "F.Cu" "B.Cu") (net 6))
 (via (at 137.609868 110.475987) (size 0.6) (drill 0.3) (layers "F.Cu" "B.Cu") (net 6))
 (via (at 134 118.5) (size 0.6) (drill 0.3) (layers "F.Cu" "B.Cu") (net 6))
 (via (at 136.259868 110.475987) (size 0.6) (drill 0.3) (layers "F.Cu" "B.Cu") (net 6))
 (via (at 133.2 95.35) (size 0.6) (drill 0.3) (layers "F.Cu" "B.Cu") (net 6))
 (via (at 134.909868 108.975987) (size 0.6) (drill 0.3) (layers "F.Cu" "B.Cu") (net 6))
 (via (at 132.38 98.7) (size 0.6) (drill 0.3) (layers "F.Cu" "B.Cu") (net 6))
 (via (at 136.259868 107.425987) (size 0.6) (drill 0.3) (layers "F.Cu" "B.Cu") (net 6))
 (via (at 133.85 104.85) (size 0.6) (drill 0.3) (layers "F.Cu" "B.Cu") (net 6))
 (via (at 135.5 96) (size 0.6) (drill 0.3) (layers "F.Cu" "B.Cu") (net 6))
 (via (at 137.609868 107.425987) (size 0.6) (drill 0.3) (layers "F.Cu" "B.Cu") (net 6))
 (via (at 134.909868 110.475987) (size 0.6) (drill 0.3) (layers "F.Cu" "B.Cu") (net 6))
 (via (at 137.609868 108.975987) (size 0.6) (drill 0.3) (layers "F.Cu" "B.Cu") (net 6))
 (via (at 134.909868 107.425987) (size 0.6) (drill 0.3) (layers "F.Cu" "B.Cu") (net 6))
 (segment (start 135.9325 117.52) (end 136.8625 118.45) (width 0.2) (layer "F.Cu") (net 1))
 (segment (start 135.1 103.6) (end 132.75 101.25) (width 0.2) (layer "F.Cu") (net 1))
 (segment (start 135 117.52) (end 135 115.5) (width 0.2) (layer "F.Cu") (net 1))
 (segment (start 130.5 114.5) (end 130.5 103.5) (width 0.2) (layer "F.Cu") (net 1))
 (segment (start 135.1 104.85) (end 135.1 103.6) (width 0.2) (layer "F.Cu") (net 1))
 (segment (start 135 115.5) (end 131.5 115.5) (width 0.2) (layer "F.Cu") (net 1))
 (segment (start 131.5 115.5) (end 130.5 114.5) (width 0.2) (layer "F.Cu") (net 1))
 (segment (start 132.75 101.25) (end 133.5 100.5) (width 0.2) (layer "F.Cu") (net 1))
 (segment (start 133.5 100.5) (end 139 100.5) (width 0.2) (layer "F.Cu") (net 1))
 (segment (start 135 113.25) (end 135.1 113.15) (width 0.2) (layer "F.Cu") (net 1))
 (segment (start 135 115.5) (end 135 113.25) (width 0.2) (layer "F.Cu") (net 1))
 (segment (start 130.5 103.5) (end 132.75 101.25) (width 0.2) (layer "F.Cu") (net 1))
 (segment (start 135 117.52) (end 135.9325 117.52) (width 0.2) (layer "F.Cu") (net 1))
 (segment (start 133.2 97.52) (end 133.38 97.7) (width 0.2) (layer "F.Cu") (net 2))
 (segment (start 133.2 96.5) (end 133.2 97.52) (width 0.2) (layer "F.Cu") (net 2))
 (segment (start 133.38 97.7) (end 138.74 97.7) (width 0.2) (layer "F.Cu") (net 2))
 (segment (start 139 97.96) (end 136.38 95.34) (width 0.2) (layer "F.Cu") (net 2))
 (segment (start 146.20124 116.041) (end 145.25 116.99224) (width 0.2) (layer "F.Cu") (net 7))
 (segment (start 145.25 116.99224) (end 145.25 118) (width 0.2) (layer "F.Cu") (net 7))
 (segment (start 141.3 116.55) (end 139.1375 116.55) (width 0.2) (layer "F.Cu") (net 7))
 (segment (start 143.9 107.27) (end 145.051 108.421) (width 0.2) (layer "F.Cu") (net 7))
 (segment (start 147.209 116.041) (end 146.20124 116.041) (width 0.2) (layer "F.Cu") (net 7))
 (segment (start 147.799 109.299) (end 147.799 115.451) (width 0.2) (layer "F.Cu") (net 7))
 (segment (start 144.5 118.75) (end 143.5 118.75) (width 0.2) (layer "F.Cu") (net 7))
 (segment (start 145.25 118) (end 144.5 118.75) (width 0.2) (layer "F.Cu") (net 7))
 (segment (start 143.5 118.75) (end 141.3 116.55) (width 0.2) (layer "F.Cu") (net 7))
 (segment (start 147.799 115.451) (end 147.209 116.041) (width 0.2) (layer "F.Cu") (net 7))
 (segment (start 146.921 108.421) (end 147.799 109.299) (width 0.2) (layer "F.Cu") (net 7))
 (segment (start 145.051 108.421) (end 146.921 108.421) (width 0.2) (layer "F.Cu") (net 7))
 (segment (start 135.38 94.22) (end 134.02 94.22) (width 0.2) (layer "F.Cu") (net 4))
 (segment (start 136.38 94.2) (end 135.4 94.2) (width 0.2) (layer "F.Cu") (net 4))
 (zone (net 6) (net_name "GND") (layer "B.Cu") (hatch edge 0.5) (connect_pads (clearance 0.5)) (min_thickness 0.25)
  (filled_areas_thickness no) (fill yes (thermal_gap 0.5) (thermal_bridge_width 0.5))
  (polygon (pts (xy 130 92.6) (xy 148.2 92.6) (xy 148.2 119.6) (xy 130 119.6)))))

